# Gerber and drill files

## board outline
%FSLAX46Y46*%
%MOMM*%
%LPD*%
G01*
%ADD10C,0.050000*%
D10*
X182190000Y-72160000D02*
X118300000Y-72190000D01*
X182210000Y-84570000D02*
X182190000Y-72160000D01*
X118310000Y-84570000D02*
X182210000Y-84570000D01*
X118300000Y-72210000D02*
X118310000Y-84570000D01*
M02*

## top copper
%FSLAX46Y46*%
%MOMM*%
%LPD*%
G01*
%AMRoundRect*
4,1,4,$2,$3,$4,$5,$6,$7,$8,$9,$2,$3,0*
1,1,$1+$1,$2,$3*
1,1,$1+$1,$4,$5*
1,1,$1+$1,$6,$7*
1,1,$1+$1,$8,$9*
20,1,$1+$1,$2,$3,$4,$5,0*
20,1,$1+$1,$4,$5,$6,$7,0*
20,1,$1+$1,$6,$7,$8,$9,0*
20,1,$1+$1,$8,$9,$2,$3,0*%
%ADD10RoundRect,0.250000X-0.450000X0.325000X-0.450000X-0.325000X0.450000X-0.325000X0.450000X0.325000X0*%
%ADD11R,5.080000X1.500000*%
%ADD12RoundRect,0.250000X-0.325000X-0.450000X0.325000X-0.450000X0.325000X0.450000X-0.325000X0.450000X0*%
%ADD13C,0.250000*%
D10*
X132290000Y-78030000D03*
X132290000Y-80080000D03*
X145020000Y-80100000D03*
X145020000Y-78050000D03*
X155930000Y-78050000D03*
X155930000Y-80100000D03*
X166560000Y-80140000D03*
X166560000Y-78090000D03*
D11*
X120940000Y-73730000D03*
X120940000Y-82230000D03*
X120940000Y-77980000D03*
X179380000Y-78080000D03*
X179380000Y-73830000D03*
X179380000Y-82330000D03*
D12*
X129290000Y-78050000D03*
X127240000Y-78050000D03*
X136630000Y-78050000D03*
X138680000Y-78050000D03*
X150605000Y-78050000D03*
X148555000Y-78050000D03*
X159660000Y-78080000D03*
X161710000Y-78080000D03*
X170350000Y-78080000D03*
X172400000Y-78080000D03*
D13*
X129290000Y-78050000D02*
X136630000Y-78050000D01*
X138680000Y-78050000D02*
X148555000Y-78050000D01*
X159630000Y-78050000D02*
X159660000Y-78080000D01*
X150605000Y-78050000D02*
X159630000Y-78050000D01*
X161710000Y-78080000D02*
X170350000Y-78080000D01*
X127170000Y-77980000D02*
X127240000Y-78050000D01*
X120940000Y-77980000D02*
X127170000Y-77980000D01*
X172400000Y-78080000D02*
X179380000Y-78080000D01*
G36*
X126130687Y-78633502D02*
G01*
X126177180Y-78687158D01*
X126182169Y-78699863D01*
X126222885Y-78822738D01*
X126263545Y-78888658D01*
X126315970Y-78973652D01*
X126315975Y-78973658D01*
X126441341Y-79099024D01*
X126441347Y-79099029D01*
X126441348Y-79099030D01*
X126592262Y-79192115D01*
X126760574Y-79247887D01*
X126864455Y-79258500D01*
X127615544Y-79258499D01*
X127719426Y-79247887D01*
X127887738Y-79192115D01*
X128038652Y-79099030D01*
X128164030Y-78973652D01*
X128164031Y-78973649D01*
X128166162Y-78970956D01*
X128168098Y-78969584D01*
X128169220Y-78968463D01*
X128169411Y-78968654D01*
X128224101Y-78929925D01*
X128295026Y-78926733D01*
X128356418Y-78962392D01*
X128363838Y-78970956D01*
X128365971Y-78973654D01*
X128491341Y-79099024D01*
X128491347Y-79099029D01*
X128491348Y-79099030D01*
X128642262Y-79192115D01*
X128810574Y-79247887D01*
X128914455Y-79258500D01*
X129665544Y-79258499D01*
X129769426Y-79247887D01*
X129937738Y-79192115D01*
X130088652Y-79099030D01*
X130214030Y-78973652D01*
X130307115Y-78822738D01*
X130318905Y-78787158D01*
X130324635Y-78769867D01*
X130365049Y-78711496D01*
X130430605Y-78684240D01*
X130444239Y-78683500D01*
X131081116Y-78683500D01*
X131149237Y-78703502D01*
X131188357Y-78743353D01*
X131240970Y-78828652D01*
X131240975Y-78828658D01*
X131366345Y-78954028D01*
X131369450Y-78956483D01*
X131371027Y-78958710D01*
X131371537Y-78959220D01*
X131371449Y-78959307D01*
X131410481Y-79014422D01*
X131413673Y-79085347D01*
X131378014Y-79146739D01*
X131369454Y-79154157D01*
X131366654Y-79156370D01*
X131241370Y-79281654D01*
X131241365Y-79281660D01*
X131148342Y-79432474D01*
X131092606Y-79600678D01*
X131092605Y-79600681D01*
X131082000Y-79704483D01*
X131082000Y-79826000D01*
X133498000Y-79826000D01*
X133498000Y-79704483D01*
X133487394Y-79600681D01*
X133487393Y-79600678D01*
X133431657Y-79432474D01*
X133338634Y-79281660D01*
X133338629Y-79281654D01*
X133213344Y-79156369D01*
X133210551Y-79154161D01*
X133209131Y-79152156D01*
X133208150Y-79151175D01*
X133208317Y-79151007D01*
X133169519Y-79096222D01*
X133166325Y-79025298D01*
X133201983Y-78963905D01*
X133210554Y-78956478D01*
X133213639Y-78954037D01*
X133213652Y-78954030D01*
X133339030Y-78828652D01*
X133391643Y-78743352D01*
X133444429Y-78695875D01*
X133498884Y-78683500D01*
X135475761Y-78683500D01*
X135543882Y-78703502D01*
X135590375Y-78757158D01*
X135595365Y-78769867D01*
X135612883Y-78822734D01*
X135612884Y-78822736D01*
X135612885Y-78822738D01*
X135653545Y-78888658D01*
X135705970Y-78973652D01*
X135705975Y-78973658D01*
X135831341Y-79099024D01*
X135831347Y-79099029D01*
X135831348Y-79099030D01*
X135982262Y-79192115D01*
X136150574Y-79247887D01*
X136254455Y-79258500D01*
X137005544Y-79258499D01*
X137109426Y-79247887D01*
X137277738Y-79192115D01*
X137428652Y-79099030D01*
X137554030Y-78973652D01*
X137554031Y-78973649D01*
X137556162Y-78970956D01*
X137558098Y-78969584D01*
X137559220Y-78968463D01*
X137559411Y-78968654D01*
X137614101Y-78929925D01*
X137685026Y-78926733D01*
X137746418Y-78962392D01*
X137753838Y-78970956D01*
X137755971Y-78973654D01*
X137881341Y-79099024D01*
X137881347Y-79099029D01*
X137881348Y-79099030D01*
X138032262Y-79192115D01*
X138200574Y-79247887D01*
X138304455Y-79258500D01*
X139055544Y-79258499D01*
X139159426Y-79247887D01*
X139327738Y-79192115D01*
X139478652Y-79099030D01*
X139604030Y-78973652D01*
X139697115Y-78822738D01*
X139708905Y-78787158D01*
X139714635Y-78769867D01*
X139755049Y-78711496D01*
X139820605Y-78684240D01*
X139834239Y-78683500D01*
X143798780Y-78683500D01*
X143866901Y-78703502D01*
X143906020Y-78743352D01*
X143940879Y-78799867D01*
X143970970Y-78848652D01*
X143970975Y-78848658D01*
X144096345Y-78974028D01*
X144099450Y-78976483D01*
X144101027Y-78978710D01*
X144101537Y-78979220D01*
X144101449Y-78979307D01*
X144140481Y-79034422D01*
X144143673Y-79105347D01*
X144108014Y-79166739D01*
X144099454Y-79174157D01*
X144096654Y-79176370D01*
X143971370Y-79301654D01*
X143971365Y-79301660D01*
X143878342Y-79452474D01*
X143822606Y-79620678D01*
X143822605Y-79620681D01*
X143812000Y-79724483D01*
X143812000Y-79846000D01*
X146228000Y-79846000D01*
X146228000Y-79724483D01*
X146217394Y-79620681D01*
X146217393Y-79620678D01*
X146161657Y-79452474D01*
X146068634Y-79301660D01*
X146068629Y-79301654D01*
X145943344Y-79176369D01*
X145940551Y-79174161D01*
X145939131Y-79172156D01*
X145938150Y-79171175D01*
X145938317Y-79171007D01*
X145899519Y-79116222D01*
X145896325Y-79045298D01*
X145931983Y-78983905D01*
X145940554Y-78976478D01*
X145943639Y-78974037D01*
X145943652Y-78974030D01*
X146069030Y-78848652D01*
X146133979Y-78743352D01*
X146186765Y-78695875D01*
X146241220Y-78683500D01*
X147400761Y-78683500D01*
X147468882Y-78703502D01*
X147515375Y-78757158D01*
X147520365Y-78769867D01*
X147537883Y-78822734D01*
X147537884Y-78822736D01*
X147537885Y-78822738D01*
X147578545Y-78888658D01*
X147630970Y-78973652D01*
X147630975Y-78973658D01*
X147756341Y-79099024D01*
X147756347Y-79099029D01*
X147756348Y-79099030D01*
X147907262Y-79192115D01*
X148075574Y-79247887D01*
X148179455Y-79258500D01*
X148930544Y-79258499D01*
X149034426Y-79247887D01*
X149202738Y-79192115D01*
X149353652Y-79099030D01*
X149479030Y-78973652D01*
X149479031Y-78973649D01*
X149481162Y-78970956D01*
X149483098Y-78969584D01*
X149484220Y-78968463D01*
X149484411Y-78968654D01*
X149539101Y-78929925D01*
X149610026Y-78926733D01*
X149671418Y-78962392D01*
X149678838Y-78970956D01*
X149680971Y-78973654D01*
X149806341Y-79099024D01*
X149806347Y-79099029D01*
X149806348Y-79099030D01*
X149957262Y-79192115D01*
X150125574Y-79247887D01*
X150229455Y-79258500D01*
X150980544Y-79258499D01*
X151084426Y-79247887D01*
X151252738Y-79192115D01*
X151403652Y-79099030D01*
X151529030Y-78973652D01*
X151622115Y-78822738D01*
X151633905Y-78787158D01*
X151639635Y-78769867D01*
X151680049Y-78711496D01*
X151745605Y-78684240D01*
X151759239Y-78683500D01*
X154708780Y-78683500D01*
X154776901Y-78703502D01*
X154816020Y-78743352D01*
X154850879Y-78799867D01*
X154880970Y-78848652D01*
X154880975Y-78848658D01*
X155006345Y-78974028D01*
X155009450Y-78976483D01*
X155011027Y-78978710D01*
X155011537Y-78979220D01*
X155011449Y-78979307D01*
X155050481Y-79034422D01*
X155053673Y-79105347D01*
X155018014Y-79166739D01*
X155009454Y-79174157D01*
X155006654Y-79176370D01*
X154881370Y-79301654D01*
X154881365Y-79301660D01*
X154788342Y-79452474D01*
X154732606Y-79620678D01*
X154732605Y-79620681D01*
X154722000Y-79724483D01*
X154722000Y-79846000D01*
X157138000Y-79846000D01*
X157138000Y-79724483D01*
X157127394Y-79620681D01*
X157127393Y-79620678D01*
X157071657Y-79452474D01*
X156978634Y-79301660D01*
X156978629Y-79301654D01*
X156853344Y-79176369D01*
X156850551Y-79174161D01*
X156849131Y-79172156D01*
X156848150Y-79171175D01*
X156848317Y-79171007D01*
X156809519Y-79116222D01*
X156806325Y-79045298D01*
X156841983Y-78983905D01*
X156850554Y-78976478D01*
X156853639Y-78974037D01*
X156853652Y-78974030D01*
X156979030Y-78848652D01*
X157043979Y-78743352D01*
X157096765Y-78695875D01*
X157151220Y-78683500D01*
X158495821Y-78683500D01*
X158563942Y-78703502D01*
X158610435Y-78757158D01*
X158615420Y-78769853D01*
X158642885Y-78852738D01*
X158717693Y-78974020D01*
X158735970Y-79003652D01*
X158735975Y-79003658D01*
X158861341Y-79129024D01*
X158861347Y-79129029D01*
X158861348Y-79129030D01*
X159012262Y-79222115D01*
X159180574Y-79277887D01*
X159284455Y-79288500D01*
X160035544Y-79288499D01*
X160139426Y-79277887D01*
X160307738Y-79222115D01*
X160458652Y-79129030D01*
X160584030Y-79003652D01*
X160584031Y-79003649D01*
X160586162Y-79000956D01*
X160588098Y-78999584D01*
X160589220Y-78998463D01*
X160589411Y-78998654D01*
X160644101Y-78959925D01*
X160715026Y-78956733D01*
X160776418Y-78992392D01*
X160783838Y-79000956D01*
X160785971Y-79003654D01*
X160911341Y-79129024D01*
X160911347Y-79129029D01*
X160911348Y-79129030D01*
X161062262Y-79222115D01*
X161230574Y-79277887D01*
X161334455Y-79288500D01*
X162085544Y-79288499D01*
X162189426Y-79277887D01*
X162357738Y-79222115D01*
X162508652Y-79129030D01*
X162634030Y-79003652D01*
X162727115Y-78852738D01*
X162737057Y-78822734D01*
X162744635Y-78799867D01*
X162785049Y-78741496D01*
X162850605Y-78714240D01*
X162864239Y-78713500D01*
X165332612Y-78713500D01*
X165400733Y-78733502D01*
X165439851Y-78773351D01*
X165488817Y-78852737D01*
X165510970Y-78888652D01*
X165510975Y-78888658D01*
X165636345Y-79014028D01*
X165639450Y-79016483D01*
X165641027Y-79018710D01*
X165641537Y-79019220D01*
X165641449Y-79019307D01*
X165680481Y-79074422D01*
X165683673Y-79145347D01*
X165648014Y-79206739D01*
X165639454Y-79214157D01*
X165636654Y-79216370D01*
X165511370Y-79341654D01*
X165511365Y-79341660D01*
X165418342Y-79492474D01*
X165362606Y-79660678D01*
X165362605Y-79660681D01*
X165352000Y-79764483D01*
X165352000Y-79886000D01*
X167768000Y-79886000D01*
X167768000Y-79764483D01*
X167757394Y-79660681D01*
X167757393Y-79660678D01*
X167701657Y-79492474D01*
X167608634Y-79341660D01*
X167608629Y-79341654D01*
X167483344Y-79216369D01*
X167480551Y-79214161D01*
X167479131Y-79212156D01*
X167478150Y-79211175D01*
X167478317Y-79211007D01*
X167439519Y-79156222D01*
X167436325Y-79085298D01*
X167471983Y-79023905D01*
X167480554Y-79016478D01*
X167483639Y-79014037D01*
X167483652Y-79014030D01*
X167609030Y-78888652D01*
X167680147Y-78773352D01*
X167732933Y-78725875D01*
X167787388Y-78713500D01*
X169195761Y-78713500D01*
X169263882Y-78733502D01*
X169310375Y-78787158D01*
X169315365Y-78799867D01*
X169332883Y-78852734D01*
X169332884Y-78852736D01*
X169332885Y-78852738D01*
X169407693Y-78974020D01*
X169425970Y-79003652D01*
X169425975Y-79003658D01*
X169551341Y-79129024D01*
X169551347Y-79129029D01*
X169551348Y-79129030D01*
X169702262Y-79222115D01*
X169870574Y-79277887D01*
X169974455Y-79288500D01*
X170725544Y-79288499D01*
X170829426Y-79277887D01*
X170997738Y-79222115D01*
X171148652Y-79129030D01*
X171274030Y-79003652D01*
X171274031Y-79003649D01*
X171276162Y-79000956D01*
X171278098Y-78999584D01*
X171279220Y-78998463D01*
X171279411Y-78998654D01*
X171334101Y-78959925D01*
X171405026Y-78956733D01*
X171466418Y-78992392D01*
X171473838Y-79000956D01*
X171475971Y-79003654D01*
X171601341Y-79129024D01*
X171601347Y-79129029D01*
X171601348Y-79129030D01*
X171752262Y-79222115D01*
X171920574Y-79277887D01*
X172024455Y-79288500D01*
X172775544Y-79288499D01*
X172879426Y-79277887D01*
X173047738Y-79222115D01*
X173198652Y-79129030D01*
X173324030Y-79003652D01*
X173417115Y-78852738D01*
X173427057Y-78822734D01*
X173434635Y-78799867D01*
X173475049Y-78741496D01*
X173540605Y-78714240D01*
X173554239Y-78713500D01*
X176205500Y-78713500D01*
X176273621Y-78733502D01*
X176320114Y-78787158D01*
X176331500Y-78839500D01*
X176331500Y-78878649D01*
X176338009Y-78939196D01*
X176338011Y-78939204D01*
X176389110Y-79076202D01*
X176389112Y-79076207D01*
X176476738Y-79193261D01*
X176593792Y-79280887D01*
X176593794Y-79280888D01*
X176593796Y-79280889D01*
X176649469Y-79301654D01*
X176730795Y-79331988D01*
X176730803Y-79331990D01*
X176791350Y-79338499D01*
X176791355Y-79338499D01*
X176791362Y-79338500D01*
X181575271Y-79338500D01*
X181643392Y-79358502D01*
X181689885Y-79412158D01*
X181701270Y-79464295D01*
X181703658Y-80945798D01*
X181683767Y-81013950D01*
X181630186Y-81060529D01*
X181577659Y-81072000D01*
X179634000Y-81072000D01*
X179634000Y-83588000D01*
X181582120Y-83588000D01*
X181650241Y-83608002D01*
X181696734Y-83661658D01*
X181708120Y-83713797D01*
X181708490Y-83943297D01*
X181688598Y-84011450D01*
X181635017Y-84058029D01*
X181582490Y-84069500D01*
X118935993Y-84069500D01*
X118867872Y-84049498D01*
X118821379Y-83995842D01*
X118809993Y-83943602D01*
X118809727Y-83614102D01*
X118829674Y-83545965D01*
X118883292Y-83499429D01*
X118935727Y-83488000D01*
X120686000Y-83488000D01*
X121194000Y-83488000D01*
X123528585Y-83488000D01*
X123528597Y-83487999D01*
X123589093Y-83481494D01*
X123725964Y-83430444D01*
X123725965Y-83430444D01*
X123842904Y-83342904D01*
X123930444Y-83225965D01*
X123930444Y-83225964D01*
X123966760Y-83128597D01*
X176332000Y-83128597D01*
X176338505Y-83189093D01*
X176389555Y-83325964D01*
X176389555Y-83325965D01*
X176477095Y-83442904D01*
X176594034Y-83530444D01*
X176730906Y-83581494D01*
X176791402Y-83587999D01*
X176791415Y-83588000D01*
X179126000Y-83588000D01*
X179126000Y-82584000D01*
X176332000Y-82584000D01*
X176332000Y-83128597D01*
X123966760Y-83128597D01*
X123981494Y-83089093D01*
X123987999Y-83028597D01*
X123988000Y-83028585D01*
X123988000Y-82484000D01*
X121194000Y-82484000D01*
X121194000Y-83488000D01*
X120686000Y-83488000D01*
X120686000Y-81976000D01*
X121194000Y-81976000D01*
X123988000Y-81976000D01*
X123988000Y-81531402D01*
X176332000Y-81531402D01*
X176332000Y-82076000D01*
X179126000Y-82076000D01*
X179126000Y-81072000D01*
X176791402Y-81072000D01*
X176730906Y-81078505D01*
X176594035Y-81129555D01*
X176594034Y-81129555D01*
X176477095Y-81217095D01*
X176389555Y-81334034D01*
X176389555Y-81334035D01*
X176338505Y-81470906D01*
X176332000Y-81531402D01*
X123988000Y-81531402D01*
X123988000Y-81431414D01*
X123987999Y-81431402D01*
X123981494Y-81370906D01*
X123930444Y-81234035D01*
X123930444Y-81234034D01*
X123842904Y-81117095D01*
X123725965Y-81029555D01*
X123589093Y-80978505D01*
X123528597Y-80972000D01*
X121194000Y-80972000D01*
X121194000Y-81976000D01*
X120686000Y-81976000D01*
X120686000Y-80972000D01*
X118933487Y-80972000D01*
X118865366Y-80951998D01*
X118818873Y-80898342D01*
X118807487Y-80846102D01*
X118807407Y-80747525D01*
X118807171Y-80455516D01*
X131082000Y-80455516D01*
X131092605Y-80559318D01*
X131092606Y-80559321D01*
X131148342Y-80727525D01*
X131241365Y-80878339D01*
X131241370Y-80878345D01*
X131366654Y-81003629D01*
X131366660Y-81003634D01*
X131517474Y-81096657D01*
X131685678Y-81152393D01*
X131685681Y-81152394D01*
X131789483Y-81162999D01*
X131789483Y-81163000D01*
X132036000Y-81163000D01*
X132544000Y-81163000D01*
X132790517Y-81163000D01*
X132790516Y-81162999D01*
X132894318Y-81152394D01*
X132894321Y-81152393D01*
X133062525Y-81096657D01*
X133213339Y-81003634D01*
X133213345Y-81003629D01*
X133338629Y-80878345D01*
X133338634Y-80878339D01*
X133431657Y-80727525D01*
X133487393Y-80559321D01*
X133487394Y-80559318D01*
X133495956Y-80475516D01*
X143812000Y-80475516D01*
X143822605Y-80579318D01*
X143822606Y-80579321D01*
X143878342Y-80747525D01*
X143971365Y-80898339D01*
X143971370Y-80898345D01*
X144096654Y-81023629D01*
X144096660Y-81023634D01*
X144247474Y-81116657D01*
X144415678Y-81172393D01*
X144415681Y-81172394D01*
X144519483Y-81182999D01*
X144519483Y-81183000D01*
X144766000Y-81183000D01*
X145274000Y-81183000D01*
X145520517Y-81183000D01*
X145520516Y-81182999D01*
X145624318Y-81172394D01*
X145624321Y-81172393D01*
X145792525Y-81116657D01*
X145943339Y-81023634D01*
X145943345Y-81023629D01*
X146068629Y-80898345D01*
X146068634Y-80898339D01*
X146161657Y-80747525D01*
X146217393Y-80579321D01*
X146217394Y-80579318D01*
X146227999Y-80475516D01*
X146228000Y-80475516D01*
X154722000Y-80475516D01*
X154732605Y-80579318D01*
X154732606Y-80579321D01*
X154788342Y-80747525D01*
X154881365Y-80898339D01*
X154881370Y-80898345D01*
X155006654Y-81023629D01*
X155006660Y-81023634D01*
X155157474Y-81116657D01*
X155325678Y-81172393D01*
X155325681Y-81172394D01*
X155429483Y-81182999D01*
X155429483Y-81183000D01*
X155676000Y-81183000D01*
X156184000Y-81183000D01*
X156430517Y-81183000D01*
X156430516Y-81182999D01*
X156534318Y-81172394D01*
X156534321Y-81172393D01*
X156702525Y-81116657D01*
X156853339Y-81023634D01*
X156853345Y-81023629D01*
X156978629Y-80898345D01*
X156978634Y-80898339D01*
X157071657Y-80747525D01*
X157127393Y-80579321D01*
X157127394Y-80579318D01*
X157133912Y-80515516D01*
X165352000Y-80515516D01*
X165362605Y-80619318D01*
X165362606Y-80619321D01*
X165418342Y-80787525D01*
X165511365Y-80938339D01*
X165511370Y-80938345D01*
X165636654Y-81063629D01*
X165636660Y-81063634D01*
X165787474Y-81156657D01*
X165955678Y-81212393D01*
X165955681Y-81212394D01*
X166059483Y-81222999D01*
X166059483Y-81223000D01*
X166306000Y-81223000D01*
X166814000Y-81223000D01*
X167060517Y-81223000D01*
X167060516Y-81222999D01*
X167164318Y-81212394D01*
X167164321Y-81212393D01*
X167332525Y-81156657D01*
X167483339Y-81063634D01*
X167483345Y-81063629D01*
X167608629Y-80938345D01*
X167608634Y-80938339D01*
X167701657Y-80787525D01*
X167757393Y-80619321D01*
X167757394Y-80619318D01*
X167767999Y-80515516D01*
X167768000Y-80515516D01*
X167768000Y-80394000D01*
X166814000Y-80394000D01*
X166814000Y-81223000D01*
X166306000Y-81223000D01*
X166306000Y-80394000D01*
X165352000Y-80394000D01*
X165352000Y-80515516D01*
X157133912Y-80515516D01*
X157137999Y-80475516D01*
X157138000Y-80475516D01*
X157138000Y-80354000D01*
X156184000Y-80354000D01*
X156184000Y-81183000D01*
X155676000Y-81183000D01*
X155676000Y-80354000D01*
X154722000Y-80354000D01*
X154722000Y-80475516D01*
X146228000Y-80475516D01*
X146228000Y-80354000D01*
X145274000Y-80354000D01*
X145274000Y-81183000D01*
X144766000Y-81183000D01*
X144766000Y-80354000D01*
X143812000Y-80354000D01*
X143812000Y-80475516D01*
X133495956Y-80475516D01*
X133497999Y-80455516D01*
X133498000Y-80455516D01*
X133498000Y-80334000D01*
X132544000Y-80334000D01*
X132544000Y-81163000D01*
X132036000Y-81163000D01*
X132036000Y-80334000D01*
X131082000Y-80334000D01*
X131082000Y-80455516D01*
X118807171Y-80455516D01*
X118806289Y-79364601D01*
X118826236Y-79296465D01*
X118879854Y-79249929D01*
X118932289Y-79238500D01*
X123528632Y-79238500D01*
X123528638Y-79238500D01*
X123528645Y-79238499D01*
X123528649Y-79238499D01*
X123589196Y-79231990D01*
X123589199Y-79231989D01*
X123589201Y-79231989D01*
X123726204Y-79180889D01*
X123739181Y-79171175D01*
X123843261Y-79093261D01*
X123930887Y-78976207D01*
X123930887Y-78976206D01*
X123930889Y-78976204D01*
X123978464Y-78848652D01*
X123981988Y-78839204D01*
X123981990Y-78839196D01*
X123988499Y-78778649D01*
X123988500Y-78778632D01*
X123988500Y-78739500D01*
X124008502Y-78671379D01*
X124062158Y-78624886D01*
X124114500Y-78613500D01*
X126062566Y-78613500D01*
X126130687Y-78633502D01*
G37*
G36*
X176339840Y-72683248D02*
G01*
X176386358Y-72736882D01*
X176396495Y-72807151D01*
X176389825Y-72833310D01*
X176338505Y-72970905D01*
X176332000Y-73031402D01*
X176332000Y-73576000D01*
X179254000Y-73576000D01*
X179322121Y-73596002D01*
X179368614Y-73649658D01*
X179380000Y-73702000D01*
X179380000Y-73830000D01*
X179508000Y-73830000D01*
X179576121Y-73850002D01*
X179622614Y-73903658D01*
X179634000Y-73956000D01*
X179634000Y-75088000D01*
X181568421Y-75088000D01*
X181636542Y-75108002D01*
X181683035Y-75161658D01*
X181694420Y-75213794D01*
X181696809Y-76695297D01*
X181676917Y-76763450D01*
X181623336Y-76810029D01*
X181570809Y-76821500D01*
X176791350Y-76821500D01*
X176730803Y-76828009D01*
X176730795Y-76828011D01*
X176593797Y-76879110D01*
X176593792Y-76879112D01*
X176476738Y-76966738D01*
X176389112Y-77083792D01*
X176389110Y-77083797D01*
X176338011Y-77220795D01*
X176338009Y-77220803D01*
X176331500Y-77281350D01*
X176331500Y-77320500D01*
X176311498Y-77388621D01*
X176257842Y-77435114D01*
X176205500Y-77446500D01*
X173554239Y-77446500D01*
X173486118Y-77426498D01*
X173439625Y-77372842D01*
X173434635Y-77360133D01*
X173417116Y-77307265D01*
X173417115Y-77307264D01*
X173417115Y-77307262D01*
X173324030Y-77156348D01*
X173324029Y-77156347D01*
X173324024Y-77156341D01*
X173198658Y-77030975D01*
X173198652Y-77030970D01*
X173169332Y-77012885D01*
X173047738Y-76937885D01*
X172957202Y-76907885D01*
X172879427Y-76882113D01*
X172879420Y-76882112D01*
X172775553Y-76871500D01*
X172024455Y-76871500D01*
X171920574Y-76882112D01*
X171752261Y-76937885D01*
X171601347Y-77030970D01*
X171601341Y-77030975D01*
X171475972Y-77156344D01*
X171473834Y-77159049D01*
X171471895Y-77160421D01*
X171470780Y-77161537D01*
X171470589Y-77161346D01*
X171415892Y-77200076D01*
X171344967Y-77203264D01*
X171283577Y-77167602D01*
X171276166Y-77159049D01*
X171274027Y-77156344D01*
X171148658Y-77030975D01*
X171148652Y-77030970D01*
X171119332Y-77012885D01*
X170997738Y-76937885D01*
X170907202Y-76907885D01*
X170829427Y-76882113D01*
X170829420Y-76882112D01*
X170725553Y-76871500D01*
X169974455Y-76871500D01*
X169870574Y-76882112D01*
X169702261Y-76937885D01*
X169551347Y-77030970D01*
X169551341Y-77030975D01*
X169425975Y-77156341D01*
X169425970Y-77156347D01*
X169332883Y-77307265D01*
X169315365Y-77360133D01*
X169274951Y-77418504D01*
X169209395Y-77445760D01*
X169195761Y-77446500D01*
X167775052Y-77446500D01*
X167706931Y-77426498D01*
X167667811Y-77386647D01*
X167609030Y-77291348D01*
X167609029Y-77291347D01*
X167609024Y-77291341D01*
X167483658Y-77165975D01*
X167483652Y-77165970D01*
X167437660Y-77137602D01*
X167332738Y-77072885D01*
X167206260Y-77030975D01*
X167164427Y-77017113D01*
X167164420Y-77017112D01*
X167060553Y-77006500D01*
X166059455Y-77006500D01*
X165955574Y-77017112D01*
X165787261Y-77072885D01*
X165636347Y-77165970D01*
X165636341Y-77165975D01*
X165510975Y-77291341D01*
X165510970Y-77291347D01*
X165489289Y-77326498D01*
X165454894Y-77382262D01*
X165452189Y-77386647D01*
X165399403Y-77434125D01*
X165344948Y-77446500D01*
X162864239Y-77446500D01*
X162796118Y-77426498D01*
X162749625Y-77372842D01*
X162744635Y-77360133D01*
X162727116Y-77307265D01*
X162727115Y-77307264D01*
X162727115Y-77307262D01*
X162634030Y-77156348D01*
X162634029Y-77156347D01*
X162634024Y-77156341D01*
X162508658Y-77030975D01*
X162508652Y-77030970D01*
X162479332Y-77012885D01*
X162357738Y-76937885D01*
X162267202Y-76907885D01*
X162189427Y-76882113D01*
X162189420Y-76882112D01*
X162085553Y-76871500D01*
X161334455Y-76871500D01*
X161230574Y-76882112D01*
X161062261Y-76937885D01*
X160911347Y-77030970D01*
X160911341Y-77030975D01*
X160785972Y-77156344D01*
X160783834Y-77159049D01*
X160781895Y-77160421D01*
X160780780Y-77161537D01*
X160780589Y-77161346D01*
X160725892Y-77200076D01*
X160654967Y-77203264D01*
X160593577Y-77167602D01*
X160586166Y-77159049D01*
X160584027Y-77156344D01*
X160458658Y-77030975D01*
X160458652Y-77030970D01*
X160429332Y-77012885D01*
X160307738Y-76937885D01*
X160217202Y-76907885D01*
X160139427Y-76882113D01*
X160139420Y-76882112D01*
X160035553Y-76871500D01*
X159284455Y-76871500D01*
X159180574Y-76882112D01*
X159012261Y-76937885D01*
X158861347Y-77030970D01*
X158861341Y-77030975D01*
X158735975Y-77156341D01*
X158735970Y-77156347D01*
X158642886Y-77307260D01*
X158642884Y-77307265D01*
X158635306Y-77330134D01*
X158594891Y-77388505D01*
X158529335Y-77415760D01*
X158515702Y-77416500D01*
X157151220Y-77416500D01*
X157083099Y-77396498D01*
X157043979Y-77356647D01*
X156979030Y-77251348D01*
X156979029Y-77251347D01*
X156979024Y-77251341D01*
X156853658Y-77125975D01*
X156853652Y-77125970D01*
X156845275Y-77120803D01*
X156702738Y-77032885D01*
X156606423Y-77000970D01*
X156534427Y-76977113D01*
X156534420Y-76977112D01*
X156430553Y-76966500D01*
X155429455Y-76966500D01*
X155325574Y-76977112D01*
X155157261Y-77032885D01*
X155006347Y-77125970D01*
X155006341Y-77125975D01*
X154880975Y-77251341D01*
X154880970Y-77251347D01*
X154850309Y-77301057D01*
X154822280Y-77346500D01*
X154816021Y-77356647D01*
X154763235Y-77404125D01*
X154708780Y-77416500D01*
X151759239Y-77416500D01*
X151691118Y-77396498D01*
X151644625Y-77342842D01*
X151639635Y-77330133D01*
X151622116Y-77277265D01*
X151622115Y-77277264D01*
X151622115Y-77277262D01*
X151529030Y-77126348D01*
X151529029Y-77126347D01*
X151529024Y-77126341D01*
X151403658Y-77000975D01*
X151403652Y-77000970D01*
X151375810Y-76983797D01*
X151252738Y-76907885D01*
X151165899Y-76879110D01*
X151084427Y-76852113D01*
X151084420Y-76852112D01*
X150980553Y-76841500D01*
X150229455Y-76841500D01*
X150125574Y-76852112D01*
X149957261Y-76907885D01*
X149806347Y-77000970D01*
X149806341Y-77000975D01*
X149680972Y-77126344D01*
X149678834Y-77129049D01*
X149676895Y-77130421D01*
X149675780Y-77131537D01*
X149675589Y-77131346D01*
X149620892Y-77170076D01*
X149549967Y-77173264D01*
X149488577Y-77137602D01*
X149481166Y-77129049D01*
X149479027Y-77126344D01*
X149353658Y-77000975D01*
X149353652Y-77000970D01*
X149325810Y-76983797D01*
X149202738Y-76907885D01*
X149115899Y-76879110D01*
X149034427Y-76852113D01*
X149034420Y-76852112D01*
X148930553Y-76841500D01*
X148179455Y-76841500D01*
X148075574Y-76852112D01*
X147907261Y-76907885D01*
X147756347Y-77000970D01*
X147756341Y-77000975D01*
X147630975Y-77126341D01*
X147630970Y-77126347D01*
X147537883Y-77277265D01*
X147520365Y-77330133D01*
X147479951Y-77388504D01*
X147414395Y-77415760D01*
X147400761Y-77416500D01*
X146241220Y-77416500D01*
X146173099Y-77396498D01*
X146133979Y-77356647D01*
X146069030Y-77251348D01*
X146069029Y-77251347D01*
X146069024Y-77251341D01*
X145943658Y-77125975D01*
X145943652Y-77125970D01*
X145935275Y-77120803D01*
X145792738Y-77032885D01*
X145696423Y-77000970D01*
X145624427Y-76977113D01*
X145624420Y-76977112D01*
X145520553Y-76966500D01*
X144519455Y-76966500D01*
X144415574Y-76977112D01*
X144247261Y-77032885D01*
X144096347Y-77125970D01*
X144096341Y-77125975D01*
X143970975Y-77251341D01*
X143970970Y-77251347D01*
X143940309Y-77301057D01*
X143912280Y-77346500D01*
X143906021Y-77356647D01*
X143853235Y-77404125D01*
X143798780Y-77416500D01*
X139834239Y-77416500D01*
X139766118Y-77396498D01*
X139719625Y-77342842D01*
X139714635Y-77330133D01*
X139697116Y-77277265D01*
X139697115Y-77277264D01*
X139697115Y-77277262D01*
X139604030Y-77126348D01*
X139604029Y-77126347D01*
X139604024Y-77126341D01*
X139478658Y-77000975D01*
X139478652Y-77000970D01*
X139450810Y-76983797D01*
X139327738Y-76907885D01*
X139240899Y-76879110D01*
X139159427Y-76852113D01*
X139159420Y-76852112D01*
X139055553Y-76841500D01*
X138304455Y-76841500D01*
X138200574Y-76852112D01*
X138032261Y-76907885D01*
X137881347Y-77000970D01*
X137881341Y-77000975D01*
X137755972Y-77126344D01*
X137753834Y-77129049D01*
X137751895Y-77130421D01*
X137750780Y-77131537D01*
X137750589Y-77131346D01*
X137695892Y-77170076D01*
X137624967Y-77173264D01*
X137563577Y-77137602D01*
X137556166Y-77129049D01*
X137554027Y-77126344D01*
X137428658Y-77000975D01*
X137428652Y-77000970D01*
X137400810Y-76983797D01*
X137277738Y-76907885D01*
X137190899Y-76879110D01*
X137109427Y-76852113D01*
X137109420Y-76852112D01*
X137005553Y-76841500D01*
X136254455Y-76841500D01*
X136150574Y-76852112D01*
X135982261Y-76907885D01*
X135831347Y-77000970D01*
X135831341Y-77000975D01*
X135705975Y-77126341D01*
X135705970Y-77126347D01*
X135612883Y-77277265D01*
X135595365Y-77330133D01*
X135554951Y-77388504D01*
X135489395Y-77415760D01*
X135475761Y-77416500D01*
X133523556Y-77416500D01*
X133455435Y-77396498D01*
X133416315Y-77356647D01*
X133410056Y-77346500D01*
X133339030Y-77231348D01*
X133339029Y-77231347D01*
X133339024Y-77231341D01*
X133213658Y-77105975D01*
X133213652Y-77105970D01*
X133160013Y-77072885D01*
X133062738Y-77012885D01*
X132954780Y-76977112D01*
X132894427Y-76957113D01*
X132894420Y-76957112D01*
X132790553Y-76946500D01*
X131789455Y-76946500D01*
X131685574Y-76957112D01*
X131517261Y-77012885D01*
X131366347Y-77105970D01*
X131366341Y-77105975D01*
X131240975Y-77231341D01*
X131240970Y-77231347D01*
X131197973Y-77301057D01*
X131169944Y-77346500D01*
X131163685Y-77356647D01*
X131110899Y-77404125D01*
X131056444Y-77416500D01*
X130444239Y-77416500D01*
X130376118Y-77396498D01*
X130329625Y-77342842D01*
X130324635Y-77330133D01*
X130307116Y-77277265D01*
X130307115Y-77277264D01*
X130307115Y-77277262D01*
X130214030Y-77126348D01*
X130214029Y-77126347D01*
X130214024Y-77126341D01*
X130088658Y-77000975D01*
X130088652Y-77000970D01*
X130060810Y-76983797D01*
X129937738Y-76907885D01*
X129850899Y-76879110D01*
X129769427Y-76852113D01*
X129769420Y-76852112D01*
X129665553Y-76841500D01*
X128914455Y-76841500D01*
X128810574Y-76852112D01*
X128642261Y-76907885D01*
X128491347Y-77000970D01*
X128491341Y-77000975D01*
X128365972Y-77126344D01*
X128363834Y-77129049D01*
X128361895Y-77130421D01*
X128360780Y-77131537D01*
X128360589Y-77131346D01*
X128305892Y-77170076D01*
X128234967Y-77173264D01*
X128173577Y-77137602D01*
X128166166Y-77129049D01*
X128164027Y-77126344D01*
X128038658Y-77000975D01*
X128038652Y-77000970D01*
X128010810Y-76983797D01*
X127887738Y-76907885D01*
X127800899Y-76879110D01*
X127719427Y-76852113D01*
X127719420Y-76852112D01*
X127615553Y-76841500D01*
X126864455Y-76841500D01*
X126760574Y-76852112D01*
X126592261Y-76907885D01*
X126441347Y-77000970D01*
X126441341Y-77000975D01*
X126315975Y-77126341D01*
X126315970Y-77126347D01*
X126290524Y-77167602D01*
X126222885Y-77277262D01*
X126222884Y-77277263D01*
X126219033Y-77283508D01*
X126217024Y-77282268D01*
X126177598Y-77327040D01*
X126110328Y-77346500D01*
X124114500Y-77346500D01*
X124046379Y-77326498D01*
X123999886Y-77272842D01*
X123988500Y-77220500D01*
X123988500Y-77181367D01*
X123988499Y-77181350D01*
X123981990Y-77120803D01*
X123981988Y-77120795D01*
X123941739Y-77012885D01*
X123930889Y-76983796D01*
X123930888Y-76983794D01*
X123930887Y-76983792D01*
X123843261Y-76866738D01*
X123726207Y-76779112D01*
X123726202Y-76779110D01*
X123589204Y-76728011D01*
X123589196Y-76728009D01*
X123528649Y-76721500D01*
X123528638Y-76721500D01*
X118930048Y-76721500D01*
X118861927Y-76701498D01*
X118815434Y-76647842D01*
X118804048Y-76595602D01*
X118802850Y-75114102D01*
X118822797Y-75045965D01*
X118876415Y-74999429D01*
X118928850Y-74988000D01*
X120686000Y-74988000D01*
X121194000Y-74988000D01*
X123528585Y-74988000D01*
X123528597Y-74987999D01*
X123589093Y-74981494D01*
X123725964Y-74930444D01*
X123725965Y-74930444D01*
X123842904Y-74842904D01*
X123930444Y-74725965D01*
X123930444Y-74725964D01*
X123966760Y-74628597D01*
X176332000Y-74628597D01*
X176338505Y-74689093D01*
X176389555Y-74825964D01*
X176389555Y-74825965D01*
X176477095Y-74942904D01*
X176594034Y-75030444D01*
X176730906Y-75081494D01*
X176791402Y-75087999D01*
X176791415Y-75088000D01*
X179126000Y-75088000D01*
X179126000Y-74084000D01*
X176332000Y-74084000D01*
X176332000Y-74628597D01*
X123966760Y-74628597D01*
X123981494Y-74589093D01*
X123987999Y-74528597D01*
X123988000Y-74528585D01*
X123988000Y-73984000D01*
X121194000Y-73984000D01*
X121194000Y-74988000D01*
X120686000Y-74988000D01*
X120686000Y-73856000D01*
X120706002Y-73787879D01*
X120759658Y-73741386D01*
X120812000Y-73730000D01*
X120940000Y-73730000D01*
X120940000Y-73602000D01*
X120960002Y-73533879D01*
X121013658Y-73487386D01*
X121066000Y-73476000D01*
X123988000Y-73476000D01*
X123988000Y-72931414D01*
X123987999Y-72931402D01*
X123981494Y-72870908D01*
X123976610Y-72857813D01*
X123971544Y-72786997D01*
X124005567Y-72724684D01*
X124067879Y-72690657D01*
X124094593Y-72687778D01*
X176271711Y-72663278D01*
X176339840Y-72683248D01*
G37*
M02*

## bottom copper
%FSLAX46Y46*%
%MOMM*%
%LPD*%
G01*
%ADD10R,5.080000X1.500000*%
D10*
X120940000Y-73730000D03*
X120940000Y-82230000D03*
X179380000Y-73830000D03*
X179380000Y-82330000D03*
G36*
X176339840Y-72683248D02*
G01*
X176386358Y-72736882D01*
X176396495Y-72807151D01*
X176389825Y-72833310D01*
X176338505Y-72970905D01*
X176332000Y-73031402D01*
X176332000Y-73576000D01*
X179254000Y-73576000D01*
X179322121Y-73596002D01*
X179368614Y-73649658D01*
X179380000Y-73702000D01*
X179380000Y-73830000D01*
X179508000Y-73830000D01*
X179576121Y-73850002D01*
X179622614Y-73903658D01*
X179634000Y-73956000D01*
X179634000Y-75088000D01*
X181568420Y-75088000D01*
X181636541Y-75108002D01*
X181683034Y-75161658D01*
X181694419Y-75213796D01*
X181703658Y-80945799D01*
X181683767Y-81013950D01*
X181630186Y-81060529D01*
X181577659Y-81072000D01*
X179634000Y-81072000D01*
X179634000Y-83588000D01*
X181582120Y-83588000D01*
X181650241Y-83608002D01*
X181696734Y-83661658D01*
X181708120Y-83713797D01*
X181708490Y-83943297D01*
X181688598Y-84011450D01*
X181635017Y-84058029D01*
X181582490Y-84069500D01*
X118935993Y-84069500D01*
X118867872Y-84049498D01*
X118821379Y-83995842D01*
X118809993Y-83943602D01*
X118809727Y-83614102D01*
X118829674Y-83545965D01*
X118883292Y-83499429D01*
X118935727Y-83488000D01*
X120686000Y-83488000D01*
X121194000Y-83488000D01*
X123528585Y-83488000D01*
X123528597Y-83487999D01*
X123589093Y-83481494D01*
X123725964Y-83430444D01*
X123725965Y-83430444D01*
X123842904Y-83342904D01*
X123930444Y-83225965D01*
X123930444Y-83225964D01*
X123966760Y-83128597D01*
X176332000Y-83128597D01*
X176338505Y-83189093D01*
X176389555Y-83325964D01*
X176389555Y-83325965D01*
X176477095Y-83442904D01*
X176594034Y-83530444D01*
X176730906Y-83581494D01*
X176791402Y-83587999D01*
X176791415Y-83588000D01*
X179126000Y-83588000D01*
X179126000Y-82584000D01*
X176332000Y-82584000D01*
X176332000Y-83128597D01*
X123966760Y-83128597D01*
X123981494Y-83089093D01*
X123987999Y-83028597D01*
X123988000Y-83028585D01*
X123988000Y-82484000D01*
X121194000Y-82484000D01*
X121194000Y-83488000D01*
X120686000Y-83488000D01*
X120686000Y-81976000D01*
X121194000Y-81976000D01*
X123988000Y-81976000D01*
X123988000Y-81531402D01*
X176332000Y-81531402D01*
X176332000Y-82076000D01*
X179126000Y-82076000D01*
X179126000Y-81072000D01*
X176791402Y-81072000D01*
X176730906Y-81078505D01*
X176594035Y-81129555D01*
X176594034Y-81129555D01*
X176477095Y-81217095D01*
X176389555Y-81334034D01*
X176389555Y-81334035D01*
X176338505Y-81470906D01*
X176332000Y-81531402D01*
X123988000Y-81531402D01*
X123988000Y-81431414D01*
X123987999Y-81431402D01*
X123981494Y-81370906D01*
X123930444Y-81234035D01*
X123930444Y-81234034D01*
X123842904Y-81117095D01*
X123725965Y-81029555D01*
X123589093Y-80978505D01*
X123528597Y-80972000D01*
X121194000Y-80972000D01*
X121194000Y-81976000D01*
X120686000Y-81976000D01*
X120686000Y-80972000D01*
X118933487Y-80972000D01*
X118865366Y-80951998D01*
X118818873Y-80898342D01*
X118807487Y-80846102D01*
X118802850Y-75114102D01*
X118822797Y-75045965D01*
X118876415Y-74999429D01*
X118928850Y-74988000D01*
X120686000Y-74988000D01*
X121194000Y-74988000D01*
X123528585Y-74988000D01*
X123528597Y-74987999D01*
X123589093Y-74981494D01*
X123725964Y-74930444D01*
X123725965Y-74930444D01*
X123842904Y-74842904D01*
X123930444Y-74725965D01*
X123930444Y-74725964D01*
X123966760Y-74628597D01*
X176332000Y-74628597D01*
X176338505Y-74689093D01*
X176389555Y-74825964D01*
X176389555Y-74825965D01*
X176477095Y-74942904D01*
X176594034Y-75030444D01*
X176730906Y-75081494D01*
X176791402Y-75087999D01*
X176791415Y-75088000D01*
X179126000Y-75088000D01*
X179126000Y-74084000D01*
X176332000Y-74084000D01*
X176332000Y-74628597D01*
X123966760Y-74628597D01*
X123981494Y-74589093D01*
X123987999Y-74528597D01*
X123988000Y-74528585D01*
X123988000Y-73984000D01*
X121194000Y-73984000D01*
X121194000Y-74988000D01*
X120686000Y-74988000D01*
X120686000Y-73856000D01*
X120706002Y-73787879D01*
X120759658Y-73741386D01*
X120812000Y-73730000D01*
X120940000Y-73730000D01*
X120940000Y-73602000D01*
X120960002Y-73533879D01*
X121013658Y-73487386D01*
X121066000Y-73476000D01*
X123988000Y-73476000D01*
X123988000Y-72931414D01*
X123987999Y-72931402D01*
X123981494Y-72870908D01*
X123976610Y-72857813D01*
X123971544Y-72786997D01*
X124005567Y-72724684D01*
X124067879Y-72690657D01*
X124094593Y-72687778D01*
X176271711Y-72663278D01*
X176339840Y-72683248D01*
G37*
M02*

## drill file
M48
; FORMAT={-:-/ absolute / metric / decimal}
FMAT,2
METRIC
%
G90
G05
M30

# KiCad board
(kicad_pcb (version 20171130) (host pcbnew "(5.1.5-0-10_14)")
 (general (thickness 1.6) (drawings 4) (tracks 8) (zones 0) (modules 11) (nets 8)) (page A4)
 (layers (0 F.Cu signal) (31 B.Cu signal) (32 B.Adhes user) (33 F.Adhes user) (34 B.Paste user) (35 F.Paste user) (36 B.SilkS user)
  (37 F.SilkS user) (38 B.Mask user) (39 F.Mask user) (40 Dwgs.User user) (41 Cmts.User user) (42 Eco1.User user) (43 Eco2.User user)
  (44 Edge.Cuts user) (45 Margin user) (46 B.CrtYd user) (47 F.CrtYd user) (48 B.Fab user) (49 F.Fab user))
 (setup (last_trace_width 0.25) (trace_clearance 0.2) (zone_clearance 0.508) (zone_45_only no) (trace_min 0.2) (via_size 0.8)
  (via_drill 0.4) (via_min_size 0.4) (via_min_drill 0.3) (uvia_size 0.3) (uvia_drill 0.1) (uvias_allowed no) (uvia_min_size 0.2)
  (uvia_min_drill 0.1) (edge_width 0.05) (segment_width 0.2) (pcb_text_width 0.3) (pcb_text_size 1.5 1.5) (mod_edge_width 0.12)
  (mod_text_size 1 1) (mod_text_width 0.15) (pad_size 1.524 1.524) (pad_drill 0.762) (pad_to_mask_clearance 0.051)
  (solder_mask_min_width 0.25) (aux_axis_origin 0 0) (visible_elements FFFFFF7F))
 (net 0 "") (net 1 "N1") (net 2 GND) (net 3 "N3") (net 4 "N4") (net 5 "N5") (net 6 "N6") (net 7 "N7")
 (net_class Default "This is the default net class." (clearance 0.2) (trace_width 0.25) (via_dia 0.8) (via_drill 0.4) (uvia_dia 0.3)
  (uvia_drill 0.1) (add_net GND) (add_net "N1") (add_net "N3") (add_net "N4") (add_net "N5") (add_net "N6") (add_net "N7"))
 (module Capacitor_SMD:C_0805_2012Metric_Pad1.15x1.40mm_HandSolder (layer F.Cu) (at 132.29 79.055 270)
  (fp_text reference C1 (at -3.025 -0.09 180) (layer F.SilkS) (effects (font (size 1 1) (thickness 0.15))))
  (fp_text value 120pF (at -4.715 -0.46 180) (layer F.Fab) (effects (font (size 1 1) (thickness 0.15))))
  (pad 1 smd roundrect (at -1.025 0 270) (size 1.15 1.4) (layers F.Cu F.Paste F.Mask) (roundrect_rratio 0.217391) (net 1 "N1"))
  (pad 2 smd roundrect (at 1.025 0 270) (size 1.15 1.4) (layers F.Cu F.Paste F.Mask) (roundrect_rratio 0.217391) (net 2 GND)))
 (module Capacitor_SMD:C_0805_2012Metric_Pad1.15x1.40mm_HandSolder (layer F.Cu) (at 145.02 79.075 270)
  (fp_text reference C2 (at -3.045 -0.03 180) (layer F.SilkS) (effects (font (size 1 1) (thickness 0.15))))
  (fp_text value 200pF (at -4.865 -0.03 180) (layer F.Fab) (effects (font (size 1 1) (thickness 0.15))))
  (pad 2 smd roundrect (at 1.025 0 270) (size 1.15 1.4) (layers F.Cu F.Paste F.Mask) (roundrect_rratio 0.217391) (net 2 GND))
  (pad 1 smd roundrect (at -1.025 0 270) (size 1.15 1.4) (layers F.Cu F.Paste F.Mask) (roundrect_rratio 0.217391) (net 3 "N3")))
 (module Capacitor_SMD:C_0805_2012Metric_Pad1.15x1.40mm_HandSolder (layer F.Cu) (at 155.93 79.075 270)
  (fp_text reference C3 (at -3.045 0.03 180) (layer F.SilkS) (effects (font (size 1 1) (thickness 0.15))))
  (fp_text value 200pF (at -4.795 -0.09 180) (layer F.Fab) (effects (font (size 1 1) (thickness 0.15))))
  (pad 1 smd roundrect (at -1.025 0 270) (size 1.15 1.4) (layers F.Cu F.Paste F.Mask) (roundrect_rratio 0.217391) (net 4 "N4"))
  (pad 2 smd roundrect (at 1.025 0 270) (size 1.15 1.4) (layers F.Cu F.Paste F.Mask) (roundrect_rratio 0.217391) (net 2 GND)))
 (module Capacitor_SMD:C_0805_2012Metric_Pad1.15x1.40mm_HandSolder (layer F.Cu) (at 166.56 79.115 270)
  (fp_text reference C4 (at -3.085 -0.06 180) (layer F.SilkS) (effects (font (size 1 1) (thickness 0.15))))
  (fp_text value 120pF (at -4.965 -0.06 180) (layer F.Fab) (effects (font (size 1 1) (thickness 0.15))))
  (pad 2 smd roundrect (at 1.025 0 270) (size 1.15 1.4) (layers F.Cu F.Paste F.Mask) (roundrect_rratio 0.217391) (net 2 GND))
  (pad 1 smd roundrect (at -1.025 0 270) (size 1.15 1.4) (layers F.Cu F.Paste F.Mask) (roundrect_rratio 0.217391) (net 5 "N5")))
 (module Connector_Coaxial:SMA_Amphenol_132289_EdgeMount (layer F.Cu) (at 120.94 77.98 180)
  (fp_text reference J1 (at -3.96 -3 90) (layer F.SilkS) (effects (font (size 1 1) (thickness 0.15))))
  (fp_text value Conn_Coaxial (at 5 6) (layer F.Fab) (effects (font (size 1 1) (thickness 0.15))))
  (pad 2 smd rect (at 0 4.25 270) (size 1.5 5.08) (layers B.Cu B.Paste B.Mask) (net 2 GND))
  (pad 2 smd rect (at 0 -4.25 270) (size 1.5 5.08) (layers B.Cu B.Paste B.Mask) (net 2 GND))
  (pad 2 smd rect (at 0 4.25 270) (size 1.5 5.08) (layers F.Cu F.Paste F.Mask) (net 2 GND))
  (pad 2 smd rect (at 0 -4.25 270) (size 1.5 5.08) (layers F.Cu F.Paste F.Mask) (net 2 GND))
  (pad 1 smd rect (at 0 0 270) (size 1.5 5.08) (layers F.Cu F.Paste F.Mask) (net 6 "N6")))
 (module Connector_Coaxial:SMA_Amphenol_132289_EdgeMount (layer F.Cu) (at 179.38 78.08)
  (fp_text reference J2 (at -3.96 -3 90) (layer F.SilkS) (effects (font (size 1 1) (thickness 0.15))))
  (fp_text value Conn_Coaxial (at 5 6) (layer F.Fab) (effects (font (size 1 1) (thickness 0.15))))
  (pad 1 smd rect (at 0 0 90) (size 1.5 5.08) (layers F.Cu F.Paste F.Mask) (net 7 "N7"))
  (pad 2 smd rect (at 0 -4.25 90) (size 1.5 5.08) (layers F.Cu F.Paste F.Mask) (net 2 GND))
  (pad 2 smd rect (at 0 4.25 90) (size 1.5 5.08) (layers F.Cu F.Paste F.Mask) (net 2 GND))
  (pad 2 smd rect (at 0 -4.25 90) (size 1.5 5.08) (layers B.Cu B.Paste B.Mask) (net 2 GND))
  (pad 2 smd rect (at 0 4.25 90) (size 1.5 5.08) (layers B.Cu B.Paste B.Mask) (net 2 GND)))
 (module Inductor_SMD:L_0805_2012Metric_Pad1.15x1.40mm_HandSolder (layer F.Cu) (at 128.265 78.05)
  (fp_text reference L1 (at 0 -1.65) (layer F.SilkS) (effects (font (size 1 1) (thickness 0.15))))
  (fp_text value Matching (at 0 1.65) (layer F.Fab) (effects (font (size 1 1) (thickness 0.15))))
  (pad 2 smd roundrect (at 1.025 0) (size 1.15 1.4) (layers F.Cu F.Paste F.Mask) (roundrect_rratio 0.217391) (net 1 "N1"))
  (pad 1 smd roundrect (at -1.025 0) (size 1.15 1.4) (layers F.Cu F.Paste F.Mask) (roundrect_rratio 0.217391) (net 6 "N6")))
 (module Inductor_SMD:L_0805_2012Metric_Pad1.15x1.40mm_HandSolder (layer F.Cu) (at 137.655 78.05)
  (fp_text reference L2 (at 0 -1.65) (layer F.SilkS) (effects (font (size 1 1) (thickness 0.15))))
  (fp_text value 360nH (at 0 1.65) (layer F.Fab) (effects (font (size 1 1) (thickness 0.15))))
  (pad 1 smd roundrect (at -1.025 0) (size 1.15 1.4) (layers F.Cu F.Paste F.Mask) (roundrect_rratio 0.217391) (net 1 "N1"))
  (pad 2 smd roundrect (at 1.025 0) (size 1.15 1.4) (layers F.Cu F.Paste F.Mask) (roundrect_rratio 0.217391) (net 3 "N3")))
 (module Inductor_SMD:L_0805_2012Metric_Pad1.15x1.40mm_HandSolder (layer F.Cu) (at 149.58 78.05)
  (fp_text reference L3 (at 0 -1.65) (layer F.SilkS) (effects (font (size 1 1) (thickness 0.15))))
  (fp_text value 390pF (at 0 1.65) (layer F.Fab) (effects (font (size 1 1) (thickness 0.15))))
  (pad 2 smd roundrect (at 1.025 0) (size 1.15 1.4) (layers F.Cu F.Paste F.Mask) (roundrect_rratio 0.217391) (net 4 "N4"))
  (pad 1 smd roundrect (at -1.025 0) (size 1.15 1.4) (layers F.Cu F.Paste F.Mask) (roundrect_rratio 0.217391) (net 3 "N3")))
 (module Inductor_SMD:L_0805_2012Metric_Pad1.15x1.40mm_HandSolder (layer F.Cu) (at 160.685 78.08)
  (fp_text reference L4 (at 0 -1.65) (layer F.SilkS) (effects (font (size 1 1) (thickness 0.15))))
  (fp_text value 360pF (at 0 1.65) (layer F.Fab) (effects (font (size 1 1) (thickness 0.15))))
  (pad 1 smd roundrect (at -1.025 0) (size 1.15 1.4) (layers F.Cu F.Paste F.Mask) (roundrect_rratio 0.217391) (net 4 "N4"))
  (pad 2 smd roundrect (at 1.025 0) (size 1.15 1.4) (layers F.Cu F.Paste F.Mask) (roundrect_rratio 0.217391) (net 5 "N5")))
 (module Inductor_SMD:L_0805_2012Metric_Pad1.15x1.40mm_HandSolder (layer F.Cu) (at 171.375 78.08)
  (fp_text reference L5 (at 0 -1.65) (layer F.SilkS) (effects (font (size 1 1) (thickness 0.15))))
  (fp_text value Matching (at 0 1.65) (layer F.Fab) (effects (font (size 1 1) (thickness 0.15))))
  (pad 1 smd roundrect (at -1.025 0) (size 1.15 1.4) (layers F.Cu F.Paste F.Mask) (roundrect_rratio 0.217391) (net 5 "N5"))
  (pad 2 smd roundrect (at 1.025 0) (size 1.15 1.4) (layers F.Cu F.Paste F.Mask) (roundrect_rratio 0.217391) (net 7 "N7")))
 (gr_line (start 182.19 72.16) (end 118.3 72.19) (layer Edge.Cuts) (width 0.05))
 (gr_line (start 182.21 84.57) (end 182.19 72.16) (layer Edge.Cuts) (width 0.05))
 (gr_line (start 118.31 84.57) (end 182.21 84.57) (layer Edge.Cuts) (width 0.05))
 (gr_line (start 118.3 72.21) (end 118.31 84.57) (layer Edge.Cuts) (width 0.05))
 (segment (start 129.29 78.05) (end 136.63 78.05) (width 0.25) (layer F.Cu) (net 1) (status 30))
 (segment (start 138.68 78.05) (end 148.555 78.05) (width 0.25) (layer F.Cu) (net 3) (status 30))
 (segment (start 159.63 78.05) (end 159.66 78.08) (width 0.25) (layer F.Cu) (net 4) (status 30))
 (segment (start 150.605 78.05) (end 159.63 78.05) (width 0.25) (layer F.Cu) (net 4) (status 30))
 (segment (start 161.71 78.08) (end 170.35 78.08) (width 0.25) (layer F.Cu) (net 5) (status 30))
 (segment (start 127.17 77.98) (end 127.24 78.05) (width 0.25) (layer F.Cu) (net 6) (status 30))
 (segment (start 120.94 77.98) (end 127.17 77.98) (width 0.25) (layer F.Cu) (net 6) (status 30))
 (segment (start 172.4 78.08) (end 179.38 78.08) (width 0.25) (layer F.Cu) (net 7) (status 30))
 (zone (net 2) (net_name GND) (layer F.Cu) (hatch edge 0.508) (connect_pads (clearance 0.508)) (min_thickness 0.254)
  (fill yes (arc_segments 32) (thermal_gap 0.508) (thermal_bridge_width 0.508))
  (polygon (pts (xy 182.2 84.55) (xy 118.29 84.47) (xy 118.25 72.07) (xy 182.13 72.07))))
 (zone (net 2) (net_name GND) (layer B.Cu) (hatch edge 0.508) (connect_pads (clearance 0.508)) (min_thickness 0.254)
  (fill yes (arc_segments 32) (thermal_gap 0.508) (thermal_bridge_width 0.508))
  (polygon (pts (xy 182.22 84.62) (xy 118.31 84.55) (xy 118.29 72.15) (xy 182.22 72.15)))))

